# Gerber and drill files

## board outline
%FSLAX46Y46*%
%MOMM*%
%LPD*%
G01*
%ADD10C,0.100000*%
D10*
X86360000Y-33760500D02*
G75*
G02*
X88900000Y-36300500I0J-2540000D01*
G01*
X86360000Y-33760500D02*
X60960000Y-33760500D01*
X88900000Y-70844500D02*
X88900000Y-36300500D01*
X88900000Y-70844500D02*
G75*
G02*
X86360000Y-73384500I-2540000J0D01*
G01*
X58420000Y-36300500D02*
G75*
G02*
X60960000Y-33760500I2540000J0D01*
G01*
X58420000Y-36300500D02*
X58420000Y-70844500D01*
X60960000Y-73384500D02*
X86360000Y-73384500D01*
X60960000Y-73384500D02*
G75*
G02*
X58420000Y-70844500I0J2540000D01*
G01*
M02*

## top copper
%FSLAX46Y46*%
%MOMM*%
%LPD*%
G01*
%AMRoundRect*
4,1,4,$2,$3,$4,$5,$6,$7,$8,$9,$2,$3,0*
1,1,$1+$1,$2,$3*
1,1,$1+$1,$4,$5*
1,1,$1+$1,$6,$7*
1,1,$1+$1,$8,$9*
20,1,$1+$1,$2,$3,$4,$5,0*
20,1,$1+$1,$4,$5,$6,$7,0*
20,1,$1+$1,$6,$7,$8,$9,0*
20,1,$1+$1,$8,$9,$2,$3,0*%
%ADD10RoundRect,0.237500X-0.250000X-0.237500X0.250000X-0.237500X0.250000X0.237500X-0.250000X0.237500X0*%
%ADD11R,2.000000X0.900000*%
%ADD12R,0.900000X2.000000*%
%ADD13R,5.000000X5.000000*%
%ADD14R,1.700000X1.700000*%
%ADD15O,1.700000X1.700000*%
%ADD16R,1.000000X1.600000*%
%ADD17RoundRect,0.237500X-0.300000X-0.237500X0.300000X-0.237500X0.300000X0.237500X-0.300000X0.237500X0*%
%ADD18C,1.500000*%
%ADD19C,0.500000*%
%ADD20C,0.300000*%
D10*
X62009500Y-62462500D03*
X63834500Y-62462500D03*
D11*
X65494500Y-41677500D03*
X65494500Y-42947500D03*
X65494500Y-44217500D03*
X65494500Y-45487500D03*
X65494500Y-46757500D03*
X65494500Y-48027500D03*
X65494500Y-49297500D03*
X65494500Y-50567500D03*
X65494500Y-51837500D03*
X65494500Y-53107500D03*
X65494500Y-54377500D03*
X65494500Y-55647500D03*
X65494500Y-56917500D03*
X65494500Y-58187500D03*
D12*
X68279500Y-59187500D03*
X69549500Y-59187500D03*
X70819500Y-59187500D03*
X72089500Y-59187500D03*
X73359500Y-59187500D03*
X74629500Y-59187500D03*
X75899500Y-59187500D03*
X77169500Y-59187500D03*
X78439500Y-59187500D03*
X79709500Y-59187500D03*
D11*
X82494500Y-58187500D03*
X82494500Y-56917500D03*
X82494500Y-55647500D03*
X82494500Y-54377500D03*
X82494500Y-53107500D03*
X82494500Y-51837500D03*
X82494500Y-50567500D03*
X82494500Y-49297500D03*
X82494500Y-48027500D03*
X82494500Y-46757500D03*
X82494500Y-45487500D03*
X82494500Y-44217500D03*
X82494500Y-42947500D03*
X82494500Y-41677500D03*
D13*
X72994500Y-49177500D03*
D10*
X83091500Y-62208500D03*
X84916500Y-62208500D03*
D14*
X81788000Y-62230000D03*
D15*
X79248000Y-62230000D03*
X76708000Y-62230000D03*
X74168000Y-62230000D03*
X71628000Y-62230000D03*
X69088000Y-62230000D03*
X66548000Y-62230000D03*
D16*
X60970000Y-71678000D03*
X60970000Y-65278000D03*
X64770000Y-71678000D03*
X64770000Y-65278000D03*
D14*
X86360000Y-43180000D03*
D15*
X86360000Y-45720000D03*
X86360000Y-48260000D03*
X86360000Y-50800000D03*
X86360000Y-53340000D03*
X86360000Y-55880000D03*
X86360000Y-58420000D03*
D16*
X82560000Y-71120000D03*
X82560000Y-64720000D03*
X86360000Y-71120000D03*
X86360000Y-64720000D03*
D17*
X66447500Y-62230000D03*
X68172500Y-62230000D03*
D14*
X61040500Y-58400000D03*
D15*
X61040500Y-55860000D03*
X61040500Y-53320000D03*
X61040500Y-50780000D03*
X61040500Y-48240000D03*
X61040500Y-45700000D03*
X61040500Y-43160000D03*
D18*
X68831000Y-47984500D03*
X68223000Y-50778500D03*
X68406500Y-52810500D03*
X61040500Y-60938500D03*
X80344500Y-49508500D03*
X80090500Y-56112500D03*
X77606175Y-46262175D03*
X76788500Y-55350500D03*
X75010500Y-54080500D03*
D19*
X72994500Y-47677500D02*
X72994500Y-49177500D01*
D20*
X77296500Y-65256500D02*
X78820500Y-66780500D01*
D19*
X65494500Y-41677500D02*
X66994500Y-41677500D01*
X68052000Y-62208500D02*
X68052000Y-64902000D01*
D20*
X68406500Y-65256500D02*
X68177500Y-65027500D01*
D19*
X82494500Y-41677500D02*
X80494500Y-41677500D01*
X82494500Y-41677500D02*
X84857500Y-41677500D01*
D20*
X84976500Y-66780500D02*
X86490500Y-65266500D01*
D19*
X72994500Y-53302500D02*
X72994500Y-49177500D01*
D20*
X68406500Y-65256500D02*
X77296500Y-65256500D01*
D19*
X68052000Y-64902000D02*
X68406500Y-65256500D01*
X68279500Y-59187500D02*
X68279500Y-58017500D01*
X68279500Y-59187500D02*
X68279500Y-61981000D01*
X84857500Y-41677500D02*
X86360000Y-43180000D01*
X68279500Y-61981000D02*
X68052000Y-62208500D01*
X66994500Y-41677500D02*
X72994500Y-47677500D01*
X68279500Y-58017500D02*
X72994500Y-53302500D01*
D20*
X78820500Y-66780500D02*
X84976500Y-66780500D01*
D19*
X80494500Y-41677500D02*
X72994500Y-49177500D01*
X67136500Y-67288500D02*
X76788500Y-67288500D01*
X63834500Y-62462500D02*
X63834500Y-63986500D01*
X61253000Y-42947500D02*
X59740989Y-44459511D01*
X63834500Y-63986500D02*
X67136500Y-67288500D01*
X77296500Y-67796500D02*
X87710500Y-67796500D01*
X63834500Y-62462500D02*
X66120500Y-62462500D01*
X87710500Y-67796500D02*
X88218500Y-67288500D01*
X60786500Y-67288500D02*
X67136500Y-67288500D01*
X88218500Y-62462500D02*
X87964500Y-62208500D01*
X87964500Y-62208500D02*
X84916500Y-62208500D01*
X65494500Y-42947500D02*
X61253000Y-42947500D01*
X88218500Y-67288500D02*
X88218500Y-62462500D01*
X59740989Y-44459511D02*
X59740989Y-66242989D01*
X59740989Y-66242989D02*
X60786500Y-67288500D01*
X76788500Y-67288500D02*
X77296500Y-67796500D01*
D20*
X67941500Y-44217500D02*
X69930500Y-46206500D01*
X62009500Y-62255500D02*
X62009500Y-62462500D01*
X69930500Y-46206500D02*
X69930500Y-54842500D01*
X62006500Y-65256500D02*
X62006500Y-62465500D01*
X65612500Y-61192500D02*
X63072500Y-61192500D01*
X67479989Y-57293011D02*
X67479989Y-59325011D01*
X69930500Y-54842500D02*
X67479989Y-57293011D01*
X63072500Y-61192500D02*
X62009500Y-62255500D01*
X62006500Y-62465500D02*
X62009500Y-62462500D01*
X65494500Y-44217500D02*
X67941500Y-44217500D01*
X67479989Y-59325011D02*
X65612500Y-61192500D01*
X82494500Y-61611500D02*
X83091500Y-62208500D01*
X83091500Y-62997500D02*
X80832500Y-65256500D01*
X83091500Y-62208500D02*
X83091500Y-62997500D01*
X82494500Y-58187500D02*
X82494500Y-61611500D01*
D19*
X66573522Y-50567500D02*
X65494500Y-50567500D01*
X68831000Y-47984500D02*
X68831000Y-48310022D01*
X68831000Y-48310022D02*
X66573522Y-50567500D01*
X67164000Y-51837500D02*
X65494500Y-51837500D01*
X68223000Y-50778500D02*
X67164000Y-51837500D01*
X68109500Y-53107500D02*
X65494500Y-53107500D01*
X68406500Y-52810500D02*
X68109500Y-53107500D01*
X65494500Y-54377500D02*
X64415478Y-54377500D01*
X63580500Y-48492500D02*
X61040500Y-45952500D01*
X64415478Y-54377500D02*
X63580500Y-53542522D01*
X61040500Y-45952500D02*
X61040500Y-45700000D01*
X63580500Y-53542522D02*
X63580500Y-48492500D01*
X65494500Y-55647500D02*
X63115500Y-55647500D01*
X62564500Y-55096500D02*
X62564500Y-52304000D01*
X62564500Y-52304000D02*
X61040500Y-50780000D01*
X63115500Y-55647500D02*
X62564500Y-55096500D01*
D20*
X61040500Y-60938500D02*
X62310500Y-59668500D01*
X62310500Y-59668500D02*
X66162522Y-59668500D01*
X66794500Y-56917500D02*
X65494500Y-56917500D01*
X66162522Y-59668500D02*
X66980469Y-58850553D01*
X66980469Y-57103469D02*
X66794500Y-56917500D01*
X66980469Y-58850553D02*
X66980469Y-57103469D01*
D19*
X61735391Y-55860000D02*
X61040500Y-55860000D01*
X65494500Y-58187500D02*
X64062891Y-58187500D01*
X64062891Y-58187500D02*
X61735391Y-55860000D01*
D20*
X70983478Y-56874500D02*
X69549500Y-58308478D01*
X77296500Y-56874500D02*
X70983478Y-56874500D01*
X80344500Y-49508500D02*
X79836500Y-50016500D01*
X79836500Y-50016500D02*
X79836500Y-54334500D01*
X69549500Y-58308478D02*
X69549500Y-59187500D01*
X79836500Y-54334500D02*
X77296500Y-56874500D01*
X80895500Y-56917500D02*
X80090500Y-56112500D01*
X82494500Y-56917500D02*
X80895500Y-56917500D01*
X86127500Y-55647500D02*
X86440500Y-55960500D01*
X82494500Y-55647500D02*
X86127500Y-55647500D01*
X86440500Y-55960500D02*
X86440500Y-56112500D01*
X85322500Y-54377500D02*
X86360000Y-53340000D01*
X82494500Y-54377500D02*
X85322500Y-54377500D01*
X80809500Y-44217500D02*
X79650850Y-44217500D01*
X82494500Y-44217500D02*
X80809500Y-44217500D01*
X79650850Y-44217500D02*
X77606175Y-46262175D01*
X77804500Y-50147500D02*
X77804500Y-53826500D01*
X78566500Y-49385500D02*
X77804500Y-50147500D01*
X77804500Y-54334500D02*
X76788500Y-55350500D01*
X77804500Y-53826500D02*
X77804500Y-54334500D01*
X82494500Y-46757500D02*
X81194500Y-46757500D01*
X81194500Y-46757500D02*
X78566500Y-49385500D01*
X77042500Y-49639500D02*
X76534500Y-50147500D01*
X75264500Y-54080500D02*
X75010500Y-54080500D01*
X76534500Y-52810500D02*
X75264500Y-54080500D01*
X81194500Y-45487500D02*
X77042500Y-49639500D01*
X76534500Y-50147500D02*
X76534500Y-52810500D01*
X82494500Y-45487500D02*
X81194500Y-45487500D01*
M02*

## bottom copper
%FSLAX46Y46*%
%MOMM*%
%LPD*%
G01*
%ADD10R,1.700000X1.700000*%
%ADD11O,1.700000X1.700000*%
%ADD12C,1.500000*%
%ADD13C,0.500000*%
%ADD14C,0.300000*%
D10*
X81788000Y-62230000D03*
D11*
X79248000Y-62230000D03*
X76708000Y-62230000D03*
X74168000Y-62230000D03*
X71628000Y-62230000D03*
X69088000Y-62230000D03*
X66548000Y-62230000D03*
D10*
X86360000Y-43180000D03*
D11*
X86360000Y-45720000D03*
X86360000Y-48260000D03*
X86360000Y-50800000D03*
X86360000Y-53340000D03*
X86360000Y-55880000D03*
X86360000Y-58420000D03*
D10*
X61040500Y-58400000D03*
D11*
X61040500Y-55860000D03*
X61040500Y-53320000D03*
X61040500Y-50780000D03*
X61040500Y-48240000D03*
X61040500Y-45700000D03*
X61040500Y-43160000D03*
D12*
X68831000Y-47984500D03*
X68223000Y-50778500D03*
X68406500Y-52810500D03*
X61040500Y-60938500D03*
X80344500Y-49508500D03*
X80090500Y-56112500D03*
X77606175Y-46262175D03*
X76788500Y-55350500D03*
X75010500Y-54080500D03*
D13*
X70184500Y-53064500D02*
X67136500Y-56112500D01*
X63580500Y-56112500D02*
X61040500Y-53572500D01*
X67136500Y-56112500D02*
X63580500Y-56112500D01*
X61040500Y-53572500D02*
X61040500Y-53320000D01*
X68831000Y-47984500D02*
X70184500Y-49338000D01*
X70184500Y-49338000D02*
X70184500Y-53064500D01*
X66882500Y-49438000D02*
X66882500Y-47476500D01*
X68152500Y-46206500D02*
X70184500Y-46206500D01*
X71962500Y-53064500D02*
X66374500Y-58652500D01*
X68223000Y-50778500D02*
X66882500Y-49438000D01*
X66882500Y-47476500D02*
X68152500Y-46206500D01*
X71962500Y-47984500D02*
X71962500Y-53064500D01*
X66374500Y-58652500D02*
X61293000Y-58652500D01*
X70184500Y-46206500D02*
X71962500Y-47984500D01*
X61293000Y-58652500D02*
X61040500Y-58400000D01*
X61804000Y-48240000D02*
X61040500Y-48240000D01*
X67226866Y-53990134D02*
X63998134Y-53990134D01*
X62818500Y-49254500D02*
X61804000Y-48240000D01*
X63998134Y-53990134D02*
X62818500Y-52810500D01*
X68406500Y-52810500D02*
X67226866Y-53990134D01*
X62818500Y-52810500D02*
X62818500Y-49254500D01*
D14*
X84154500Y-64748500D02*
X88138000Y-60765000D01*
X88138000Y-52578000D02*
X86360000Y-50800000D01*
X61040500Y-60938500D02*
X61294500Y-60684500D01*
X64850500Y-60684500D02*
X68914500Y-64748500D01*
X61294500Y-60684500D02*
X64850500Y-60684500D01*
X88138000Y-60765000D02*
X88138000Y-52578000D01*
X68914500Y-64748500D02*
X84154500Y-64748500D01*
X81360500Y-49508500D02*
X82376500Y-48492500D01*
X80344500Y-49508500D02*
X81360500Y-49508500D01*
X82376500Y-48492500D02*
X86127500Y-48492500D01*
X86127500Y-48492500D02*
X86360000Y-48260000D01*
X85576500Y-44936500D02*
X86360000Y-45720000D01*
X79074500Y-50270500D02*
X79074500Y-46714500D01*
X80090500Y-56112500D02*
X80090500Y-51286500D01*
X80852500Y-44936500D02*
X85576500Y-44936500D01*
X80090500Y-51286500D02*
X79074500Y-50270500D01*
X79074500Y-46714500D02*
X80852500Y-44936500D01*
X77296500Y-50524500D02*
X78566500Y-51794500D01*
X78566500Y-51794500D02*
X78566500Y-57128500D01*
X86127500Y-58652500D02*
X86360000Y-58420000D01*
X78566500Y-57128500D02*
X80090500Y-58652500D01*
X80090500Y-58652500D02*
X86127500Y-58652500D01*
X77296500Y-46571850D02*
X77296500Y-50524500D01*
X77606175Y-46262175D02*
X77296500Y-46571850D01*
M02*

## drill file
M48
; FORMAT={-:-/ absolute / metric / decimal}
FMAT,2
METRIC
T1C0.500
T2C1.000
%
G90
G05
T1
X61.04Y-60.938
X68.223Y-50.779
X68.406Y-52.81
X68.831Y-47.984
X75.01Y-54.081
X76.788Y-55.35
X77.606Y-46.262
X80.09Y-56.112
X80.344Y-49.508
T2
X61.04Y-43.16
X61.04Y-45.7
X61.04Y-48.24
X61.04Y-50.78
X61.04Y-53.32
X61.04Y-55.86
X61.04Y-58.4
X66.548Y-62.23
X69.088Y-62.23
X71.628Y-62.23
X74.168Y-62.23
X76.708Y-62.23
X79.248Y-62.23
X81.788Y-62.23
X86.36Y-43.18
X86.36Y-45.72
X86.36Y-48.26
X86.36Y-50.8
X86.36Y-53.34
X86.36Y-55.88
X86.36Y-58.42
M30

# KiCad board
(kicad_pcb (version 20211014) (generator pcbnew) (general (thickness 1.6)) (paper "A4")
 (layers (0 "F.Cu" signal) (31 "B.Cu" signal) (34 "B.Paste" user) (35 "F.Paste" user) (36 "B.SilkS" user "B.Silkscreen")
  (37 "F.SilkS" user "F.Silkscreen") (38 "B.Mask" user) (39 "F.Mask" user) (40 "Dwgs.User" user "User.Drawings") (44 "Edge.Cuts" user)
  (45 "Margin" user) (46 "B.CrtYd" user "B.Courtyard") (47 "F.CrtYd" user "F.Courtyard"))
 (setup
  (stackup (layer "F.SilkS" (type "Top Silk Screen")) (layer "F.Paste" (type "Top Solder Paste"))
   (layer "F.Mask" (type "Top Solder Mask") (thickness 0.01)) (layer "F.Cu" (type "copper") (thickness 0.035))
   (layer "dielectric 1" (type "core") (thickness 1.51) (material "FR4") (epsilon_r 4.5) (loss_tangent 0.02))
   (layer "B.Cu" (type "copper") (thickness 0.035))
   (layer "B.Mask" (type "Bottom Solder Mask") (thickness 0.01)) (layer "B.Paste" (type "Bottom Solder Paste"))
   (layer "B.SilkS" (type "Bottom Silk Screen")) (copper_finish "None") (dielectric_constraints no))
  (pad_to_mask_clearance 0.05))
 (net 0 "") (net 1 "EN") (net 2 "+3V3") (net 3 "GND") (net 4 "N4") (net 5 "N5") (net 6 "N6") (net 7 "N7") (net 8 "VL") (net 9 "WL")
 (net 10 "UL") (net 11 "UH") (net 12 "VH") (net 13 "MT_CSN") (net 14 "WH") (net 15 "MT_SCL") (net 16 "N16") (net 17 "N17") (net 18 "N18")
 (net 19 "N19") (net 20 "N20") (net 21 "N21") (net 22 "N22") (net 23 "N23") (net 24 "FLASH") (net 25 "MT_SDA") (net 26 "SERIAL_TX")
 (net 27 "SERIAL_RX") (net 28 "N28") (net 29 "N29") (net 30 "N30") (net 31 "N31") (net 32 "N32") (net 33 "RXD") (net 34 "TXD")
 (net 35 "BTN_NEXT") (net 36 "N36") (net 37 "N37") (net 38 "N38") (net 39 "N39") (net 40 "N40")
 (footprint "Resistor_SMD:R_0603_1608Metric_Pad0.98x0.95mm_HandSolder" (layer "F.Cu") (at 62.922 62.4625)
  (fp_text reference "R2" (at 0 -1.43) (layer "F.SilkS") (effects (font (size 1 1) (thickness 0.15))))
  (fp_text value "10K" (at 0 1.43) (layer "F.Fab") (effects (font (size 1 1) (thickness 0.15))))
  (pad "1" smd roundrect (at -0.9125 0) (size 0.975 0.95) (layers "F.Cu" "F.Paste" "F.Mask") (roundrect_rratio 0.25) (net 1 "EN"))
  (pad "2" smd roundrect (at 0.9125 0) (size 0.975 0.95) (layers "F.Cu" "F.Paste" "F.Mask") (roundrect_rratio 0.25) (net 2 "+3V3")))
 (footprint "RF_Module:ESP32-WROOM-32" (layer "F.Cu") (at 73.9945 49.9325)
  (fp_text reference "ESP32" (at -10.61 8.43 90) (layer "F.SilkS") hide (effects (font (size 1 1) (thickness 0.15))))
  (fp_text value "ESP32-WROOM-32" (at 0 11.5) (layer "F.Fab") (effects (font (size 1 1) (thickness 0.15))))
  (pad "1" smd rect (at -8.5 -8.255) (size 2 0.9) (layers "F.Cu" "F.Paste" "F.Mask") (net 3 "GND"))
  (pad "2" smd rect (at -8.5 -6.985) (size 2 0.9) (layers "F.Cu" "F.Paste" "F.Mask") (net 2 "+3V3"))
  (pad "3" smd rect (at -8.5 -5.715) (size 2 0.9) (layers "F.Cu" "F.Paste" "F.Mask") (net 1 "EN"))
  (pad "4" smd rect (at -8.5 -4.445) (size 2 0.9) (layers "F.Cu" "F.Paste" "F.Mask") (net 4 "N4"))
  (pad "5" smd rect (at -8.5 -3.175) (size 2 0.9) (layers "F.Cu" "F.Paste" "F.Mask") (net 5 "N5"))
  (pad "6" smd rect (at -8.5 -1.905) (size 2 0.9) (layers "F.Cu" "F.Paste" "F.Mask") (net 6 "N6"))
  (pad "7" smd rect (at -8.5 -0.635) (size 2 0.9) (layers "F.Cu" "F.Paste" "F.Mask") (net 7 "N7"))
  (pad "8" smd rect (at -8.5 0.635) (size 2 0.9) (layers "F.Cu" "F.Paste" "F.Mask") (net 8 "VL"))
  (pad "9" smd rect (at -8.5 1.905) (size 2 0.9) (layers "F.Cu" "F.Paste" "F.Mask") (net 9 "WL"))
  (pad "10" smd rect (at -8.5 3.175) (size 2 0.9) (layers "F.Cu" "F.Paste" "F.Mask") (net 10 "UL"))
  (pad "11" smd rect (at -8.5 4.445) (size 2 0.9) (layers "F.Cu" "F.Paste" "F.Mask") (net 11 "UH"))
  (pad "12" smd rect (at -8.5 5.715) (size 2 0.9) (layers "F.Cu" "F.Paste" "F.Mask") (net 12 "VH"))
  (pad "13" smd rect (at -8.5 6.985) (size 2 0.9) (layers "F.Cu" "F.Paste" "F.Mask") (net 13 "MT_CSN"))
  (pad "14" smd rect (at -8.5 8.255) (size 2 0.9) (layers "F.Cu" "F.Paste" "F.Mask") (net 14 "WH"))
  (pad "15" smd rect (at -5.715 9.255 90) (size 2 0.9) (layers "F.Cu" "F.Paste" "F.Mask") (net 3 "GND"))
  (pad "16" smd rect (at -4.445 9.255 90) (size 2 0.9) (layers "F.Cu" "F.Paste" "F.Mask") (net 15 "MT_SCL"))
  (pad "17" smd rect (at -3.175 9.255 90) (size 2 0.9) (layers "F.Cu" "F.Paste" "F.Mask") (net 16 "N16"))
  (pad "18" smd rect (at -1.905 9.255 90) (size 2 0.9) (layers "F.Cu" "F.Paste" "F.Mask") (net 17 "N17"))
  (pad "19" smd rect (at -0.635 9.255 90) (size 2 0.9) (layers "F.Cu" "F.Paste" "F.Mask") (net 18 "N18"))
  (pad "20" smd rect (at 0.635 9.255 90) (size 2 0.9) (layers "F.Cu" "F.Paste" "F.Mask") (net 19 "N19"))
  (pad "21" smd rect (at 1.905 9.255 90) (size 2 0.9) (layers "F.Cu" "F.Paste" "F.Mask") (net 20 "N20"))
  (pad "22" smd rect (at 3.175 9.255 90) (size 2 0.9) (layers "F.Cu" "F.Paste" "F.Mask") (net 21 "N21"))
  (pad "23" smd rect (at 4.445 9.255 90) (size 2 0.9) (layers "F.Cu" "F.Paste" "F.Mask") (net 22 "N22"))
  (pad "24" smd rect (at 5.715 9.255 90) (size 2 0.9) (layers "F.Cu" "F.Paste" "F.Mask") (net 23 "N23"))
  (pad "25" smd rect (at 8.5 8.255) (size 2 0.9) (layers "F.Cu" "F.Paste" "F.Mask") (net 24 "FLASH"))
  (pad "26" smd rect (at 8.5 6.985) (size 2 0.9) (layers "F.Cu" "F.Paste" "F.Mask") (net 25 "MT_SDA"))
  (pad "27" smd rect (at 8.5 5.715) (size 2 0.9) (layers "F.Cu" "F.Paste" "F.Mask") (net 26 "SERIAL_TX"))
  (pad "28" smd rect (at 8.5 4.445) (size 2 0.9) (layers "F.Cu" "F.Paste" "F.Mask") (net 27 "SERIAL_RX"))
  (pad "29" smd rect (at 8.5 3.175) (size 2 0.9) (layers "F.Cu" "F.Paste" "F.Mask") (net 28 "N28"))
  (pad "30" smd rect (at 8.5 1.905) (size 2 0.9) (layers "F.Cu" "F.Paste" "F.Mask") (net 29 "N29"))
  (pad "31" smd rect (at 8.5 0.635) (size 2 0.9) (layers "F.Cu" "F.Paste" "F.Mask") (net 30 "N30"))
  (pad "32" smd rect (at 8.5 -0.635) (size 2 0.9) (layers "F.Cu" "F.Paste" "F.Mask") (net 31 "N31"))
  (pad "33" smd rect (at 8.5 -1.905) (size 2 0.9) (layers "F.Cu" "F.Paste" "F.Mask") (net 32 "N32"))
  (pad "34" smd rect (at 8.5 -3.175) (size 2 0.9) (layers "F.Cu" "F.Paste" "F.Mask") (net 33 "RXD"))
  (pad "35" smd rect (at 8.5 -4.445) (size 2 0.9) (layers "F.Cu" "F.Paste" "F.Mask") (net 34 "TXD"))
  (pad "36" smd rect (at 8.5 -5.715) (size 2 0.9) (layers "F.Cu" "F.Paste" "F.Mask") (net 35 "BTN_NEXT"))
  (pad "37" smd rect (at 8.5 -6.985) (size 2 0.9) (layers "F.Cu" "F.Paste" "F.Mask") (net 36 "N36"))
  (pad "38" smd rect (at 8.5 -8.255) (size 2 0.9) (layers "F.Cu" "F.Paste" "F.Mask") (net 3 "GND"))
  (pad "39" smd rect (at -1 -0.755) (size 5 5) (layers "F.Cu" "F.Paste" "F.Mask") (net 3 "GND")))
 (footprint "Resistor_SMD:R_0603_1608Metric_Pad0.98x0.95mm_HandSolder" (layer "F.Cu") (at 84.004 62.2085)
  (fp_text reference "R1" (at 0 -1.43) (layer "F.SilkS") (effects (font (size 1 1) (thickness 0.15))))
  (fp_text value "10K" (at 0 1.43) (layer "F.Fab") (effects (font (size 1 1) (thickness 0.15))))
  (pad "1" smd roundrect (at -0.9125 0) (size 0.975 0.95) (layers "F.Cu" "F.Paste" "F.Mask") (roundrect_rratio 0.25) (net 24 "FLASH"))
  (pad "2" smd roundrect (at 0.9125 0) (size 0.975 0.95) (layers "F.Cu" "F.Paste" "F.Mask") (roundrect_rratio 0.25) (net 2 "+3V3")))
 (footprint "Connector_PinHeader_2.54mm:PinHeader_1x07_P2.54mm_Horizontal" (layer "F.Cu") (at 81.788 62.23 -90)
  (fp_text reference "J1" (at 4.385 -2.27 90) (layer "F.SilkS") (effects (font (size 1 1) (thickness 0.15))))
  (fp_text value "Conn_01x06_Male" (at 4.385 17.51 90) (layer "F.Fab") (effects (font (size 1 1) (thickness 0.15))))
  (pad "1" thru_hole rect (at 0 0 270) (size 1.7 1.7) (drill 1) (layers *.Cu *.Mask) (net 2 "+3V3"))
  (pad "2" thru_hole oval (at 0 2.54 270) (size 1.7 1.7) (drill 1) (layers *.Cu *.Mask) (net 34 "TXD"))
  (pad "3" thru_hole oval (at 0 5.08 270) (size 1.7 1.7) (drill 1) (layers *.Cu *.Mask) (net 33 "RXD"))
  (pad "4" thru_hole oval (at 0 7.62 270) (size 1.7 1.7) (drill 1) (layers *.Cu *.Mask) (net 1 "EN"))
  (pad "5" thru_hole oval (at 0 10.16 270) (size 1.7 1.7) (drill 1) (layers *.Cu *.Mask) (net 24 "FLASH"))
  (pad "6" thru_hole oval (at 0 12.7 270) (size 1.7 1.7) (drill 1) (layers *.Cu *.Mask) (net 3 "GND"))
  (pad "7" thru_hole oval (at 0 15.24 270) (size 1.7 1.7) (drill 1) (layers *.Cu *.Mask)))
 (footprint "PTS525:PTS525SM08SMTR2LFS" (layer "F.Cu") (at 62.87 69.128 90)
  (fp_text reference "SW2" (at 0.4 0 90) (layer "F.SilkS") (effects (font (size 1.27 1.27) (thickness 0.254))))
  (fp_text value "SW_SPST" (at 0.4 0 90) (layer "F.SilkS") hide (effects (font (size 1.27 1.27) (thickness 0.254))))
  (pad "1" smd rect locked (at -2.55 -1.9 180) (size 1 1.6) (layers "F.Cu" "F.Paste" "F.Mask") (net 1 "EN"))
  (pad "2" smd rect locked (at 3.85 -1.9 180) (size 1 1.6) (layers "F.Cu" "F.Paste" "F.Mask") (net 3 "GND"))
  (pad "3" smd rect locked (at -2.55 1.9 180) (size 1 1.6) (layers "F.Cu" "F.Paste" "F.Mask") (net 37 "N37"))
  (pad "4" smd rect locked (at 3.85 1.9 180) (size 1 1.6) (layers "F.Cu" "F.Paste" "F.Mask") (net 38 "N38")))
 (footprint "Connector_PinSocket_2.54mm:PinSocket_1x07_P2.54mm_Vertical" (layer "F.Cu") (at 86.36 43.18)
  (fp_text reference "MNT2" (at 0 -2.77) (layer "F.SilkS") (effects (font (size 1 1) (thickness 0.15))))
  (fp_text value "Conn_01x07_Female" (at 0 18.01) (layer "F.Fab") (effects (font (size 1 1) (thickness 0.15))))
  (pad "1" thru_hole rect (at 0 0) (size 1.7 1.7) (drill 1) (layers *.Cu *.Mask) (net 3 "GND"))
  (pad "2" thru_hole oval (at 0 2.54) (size 1.7 1.7) (drill 1) (layers *.Cu *.Mask) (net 25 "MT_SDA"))
  (pad "3" thru_hole oval (at 0 5.08) (size 1.7 1.7) (drill 1) (layers *.Cu *.Mask) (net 15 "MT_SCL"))
  (pad "4" thru_hole oval (at 0 7.62) (size 1.7 1.7) (drill 1) (layers *.Cu *.Mask) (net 13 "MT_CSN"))
  (pad "5" thru_hole oval (at 0 10.16) (size 1.7 1.7) (drill 1) (layers *.Cu *.Mask) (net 27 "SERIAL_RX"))
  (pad "6" thru_hole oval (at 0 12.7) (size 1.7 1.7) (drill 1) (layers *.Cu *.Mask) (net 26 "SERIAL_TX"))
  (pad "7" thru_hole oval (at 0 15.24) (size 1.7 1.7) (drill 1) (layers *.Cu *.Mask) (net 35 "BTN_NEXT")))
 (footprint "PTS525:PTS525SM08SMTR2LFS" (layer "F.Cu") (at 84.46 68.57 90)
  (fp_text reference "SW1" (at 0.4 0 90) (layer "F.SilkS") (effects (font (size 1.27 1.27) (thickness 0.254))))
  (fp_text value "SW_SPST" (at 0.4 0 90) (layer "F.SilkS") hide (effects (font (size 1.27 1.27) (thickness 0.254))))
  (pad "1" smd rect locked (at -2.55 -1.9 180) (size 1 1.6) (layers "F.Cu" "F.Paste" "F.Mask") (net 24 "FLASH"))
  (pad "2" smd rect locked (at 3.85 -1.9 180) (size 1 1.6) (layers "F.Cu" "F.Paste" "F.Mask") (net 3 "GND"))
  (pad "3" smd rect locked (at -2.55 1.9 180) (size 1 1.6) (layers "F.Cu" "F.Paste" "F.Mask") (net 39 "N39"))
  (pad "4" smd rect locked (at 3.85 1.9 180) (size 1 1.6) (layers "F.Cu" "F.Paste" "F.Mask") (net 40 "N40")))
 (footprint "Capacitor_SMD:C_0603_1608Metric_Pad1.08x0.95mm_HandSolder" (layer "F.Cu") (at 67.31 62.23)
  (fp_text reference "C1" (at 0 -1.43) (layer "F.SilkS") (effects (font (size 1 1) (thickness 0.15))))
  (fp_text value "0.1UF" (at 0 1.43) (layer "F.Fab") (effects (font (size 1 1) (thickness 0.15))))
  (pad "1" smd roundrect (at -0.8625 0) (size 1.075 0.95) (layers "F.Cu" "F.Paste" "F.Mask") (roundrect_rratio 0.25) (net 2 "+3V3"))
  (pad "2" smd roundrect (at 0.8625 0) (size 1.075 0.95) (layers "F.Cu" "F.Paste" "F.Mask") (roundrect_rratio 0.25) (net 3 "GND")))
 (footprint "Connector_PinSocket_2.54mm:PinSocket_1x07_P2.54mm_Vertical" (layer "F.Cu") (at 61.0405 58.4 180)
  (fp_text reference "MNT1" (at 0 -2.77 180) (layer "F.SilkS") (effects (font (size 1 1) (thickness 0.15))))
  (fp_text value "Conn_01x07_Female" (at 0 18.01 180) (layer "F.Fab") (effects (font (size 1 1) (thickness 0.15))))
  (pad "1" thru_hole rect (at 0 0 180) (size 1.7 1.7) (drill 1) (layers *.Cu *.Mask) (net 9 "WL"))
  (pad "2" thru_hole oval (at 0 2.54 180) (size 1.7 1.7) (drill 1) (layers *.Cu *.Mask) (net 14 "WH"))
  (pad "3" thru_hole oval (at 0 5.08 180) (size 1.7 1.7) (drill 1) (layers *.Cu *.Mask) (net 8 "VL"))
  (pad "4" thru_hole oval (at 0 7.62 180) (size 1.7 1.7) (drill 1) (layers *.Cu *.Mask) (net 12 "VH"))
  (pad "5" thru_hole oval (at 0 10.16 180) (size 1.7 1.7) (drill 1) (layers *.Cu *.Mask) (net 10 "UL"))
  (pad "6" thru_hole oval (at 0 12.7 180) (size 1.7 1.7) (drill 1) (layers *.Cu *.Mask) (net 11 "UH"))
  (pad "7" thru_hole oval (at 0 15.24 180) (size 1.7 1.7) (drill 1) (layers *.Cu *.Mask) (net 2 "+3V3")))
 (gr_arc (start 86.36 33.7605) (mid 88.156051 34.504449) (end 88.9 36.3005) (layer "Edge.Cuts") (width 0.1))
 (gr_line (start 86.36 33.7605) (end 60.96 33.7605) (layer "Edge.Cuts") (width 0.1))
 (gr_line (start 88.9 70.8445) (end 88.9 36.3005) (layer "Edge.Cuts") (width 0.1))
 (gr_arc (start 88.9 70.8445) (mid 88.156051 72.640551) (end 86.36 73.3845) (layer "Edge.Cuts") (width 0.1))
 (gr_arc (start 58.42 36.3005) (mid 59.163949 34.504449) (end 60.96 33.7605) (layer "Edge.Cuts") (width 0.1))
 (gr_line (start 58.42 36.3005) (end 58.42 70.8445) (layer "Edge.Cuts") (width 0.1))
 (gr_line (start 60.96 73.3845) (end 86.36 73.3845) (layer "Edge.Cuts") (width 0.1))
 (gr_arc (start 60.96 73.3845) (mid 59.163949 72.640551) (end 58.42 70.8445) (layer "Edge.Cuts") (width 0.1))
 (segment (start 72.9945 47.6775) (end 72.9945 49.1775) (width 0.5) (layer "F.Cu") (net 3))
 (segment (start 77.2965 65.2565) (end 78.8205 66.7805) (width 0.3) (layer "F.Cu") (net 3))
 (segment (start 65.4945 41.6775) (end 66.9945 41.6775) (width 0.5) (layer "F.Cu") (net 3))
 (segment (start 68.052 62.2085) (end 68.052 64.902) (width 0.5) (layer "F.Cu") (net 3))
 (segment (start 68.4065 65.2565) (end 68.1775 65.0275) (width 0.3) (layer "F.Cu") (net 3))
 (segment (start 82.4945 41.6775) (end 80.4945 41.6775) (width 0.5) (layer "F.Cu") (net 3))
 (segment (start 82.4945 41.6775) (end 84.8575 41.6775) (width 0.5) (layer "F.Cu") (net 3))
 (segment (start 84.9765 66.7805) (end 86.4905 65.2665) (width 0.3) (layer "F.Cu") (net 3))
 (segment (start 72.9945 53.3025) (end 72.9945 49.1775) (width 0.5) (layer "F.Cu") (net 3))
 (segment (start 68.4065 65.2565) (end 77.2965 65.2565) (width 0.3) (layer "F.Cu") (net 3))
 (segment (start 68.052 64.902) (end 68.4065 65.2565) (width 0.5) (layer "F.Cu") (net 3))
 (segment (start 68.2795 59.1875) (end 68.2795 58.0175) (width 0.5) (layer "F.Cu") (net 3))
 (segment (start 68.2795 59.1875) (end 68.2795 61.981) (width 0.5) (layer "F.Cu") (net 3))
 (segment (start 84.8575 41.6775) (end 86.36 43.18) (width 0.5) (layer "F.Cu") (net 3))
 (segment (start 68.2795 61.981) (end 68.052 62.2085) (width 0.5) (layer "F.Cu") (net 3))
 (segment (start 66.9945 41.6775) (end 72.9945 47.6775) (width 0.5) (layer "F.Cu") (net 3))
 (segment (start 68.2795 58.0175) (end 72.9945 53.3025) (width 0.5) (layer "F.Cu") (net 3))
 (segment (start 78.8205 66.7805) (end 84.9765 66.7805) (width 0.3) (layer "F.Cu") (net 3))
 (segment (start 80.4945 41.6775) (end 72.9945 49.1775) (width 0.5) (layer "F.Cu") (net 3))
 (segment (start 67.1365 67.2885) (end 76.7885 67.2885) (width 0.5) (layer "F.Cu") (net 2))
 (segment (start 63.8345 62.4625) (end 63.8345 63.9865) (width 0.5) (layer "F.Cu") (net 2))
 (segment (start 61.253 42.9475) (end 59.740989 44.459511) (width 0.5) (layer "F.Cu") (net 2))
 (segment (start 63.8345 63.9865) (end 67.1365 67.2885) (width 0.5) (layer "F.Cu") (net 2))
 (segment (start 77.2965 67.7965) (end 87.7105 67.7965) (width 0.5) (layer "F.Cu") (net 2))
 (segment (start 63.8345 62.4625) (end 66.1205 62.4625) (width 0.5) (layer "F.Cu") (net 2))
 (segment (start 87.7105 67.7965) (end 88.2185 67.2885) (width 0.5) (layer "F.Cu") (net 2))
 (segment (start 60.7865 67.2885) (end 67.1365 67.2885) (width 0.5) (layer "F.Cu") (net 2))
 (segment (start 88.2185 62.4625) (end 87.9645 62.2085) (width 0.5) (layer "F.Cu") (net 2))
 (segment (start 87.9645 62.2085) (end 84.9165 62.2085) (width 0.5) (layer "F.Cu") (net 2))
 (segment (start 65.4945 42.9475) (end 61.253 42.9475) (width 0.5) (layer "F.Cu") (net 2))
 (segment (start 88.2185 67.2885) (end 88.2185 62.4625) (width 0.5) (layer "F.Cu") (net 2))
 (segment (start 59.740989 44.459511) (end 59.740989 66.242989) (width 0.5) (layer "F.Cu") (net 2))
 (segment (start 59.740989 66.242989) (end 60.7865 67.2885) (width 0.5) (layer "F.Cu") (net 2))
 (segment (start 76.7885 67.2885) (end 77.2965 67.7965) (width 0.5) (layer "F.Cu") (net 2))
 (segment (start 67.9415 44.2175) (end 69.9305 46.2065) (width 0.3) (layer "F.Cu") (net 1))
 (segment (start 62.0095 62.2555) (end 62.0095 62.4625) (width 0.3) (layer "F.Cu") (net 1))
 (segment (start 69.9305 46.2065) (end 69.9305 54.8425) (width 0.3) (layer "F.Cu") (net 1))
 (segment (start 62.0065 65.2565) (end 62.0065 62.4655) (width 0.3) (layer "F.Cu") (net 1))
 (segment (start 65.6125 61.1925) (end 63.0725 61.1925) (width 0.3) (layer "F.Cu") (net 1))
 (segment (start 67.479989 57.293011) (end 67.479989 59.325011) (width 0.3) (layer "F.Cu") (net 1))
 (segment (start 69.9305 54.8425) (end 67.479989 57.293011) (width 0.3) (layer "F.Cu") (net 1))
 (segment (start 63.0725 61.1925) (end 62.0095 62.2555) (width 0.3) (layer "F.Cu") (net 1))
 (segment (start 62.0065 62.4655) (end 62.0095 62.4625) (width 0.3) (layer "F.Cu") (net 1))
 (segment (start 65.4945 44.2175) (end 67.9415 44.2175) (width 0.3) (layer "F.Cu") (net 1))
 (segment (start 67.479989 59.325011) (end 65.6125 61.1925) (width 0.3) (layer "F.Cu") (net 1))
 (segment (start 82.4945 61.6115) (end 83.0915 62.2085) (width 0.3) (layer "F.Cu") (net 24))
 (segment (start 83.0915 62.9975) (end 80.8325 65.2565) (width 0.3) (layer "F.Cu") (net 24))
 (segment (start 83.0915 62.2085) (end 83.0915 62.9975) (width 0.3) (layer "F.Cu") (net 24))
 (segment (start 82.4945 58.1875) (end 82.4945 61.6115) (width 0.3) (layer "F.Cu") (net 24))
 (segment (start 66.573522 50.5675) (end 65.4945 50.5675) (width 0.5) (layer "F.Cu") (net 8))
 (segment (start 68.831 47.9845) (end 68.831 48.310022) (width 0.5) (layer "F.Cu") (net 8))
 (segment (start 68.831 48.310022) (end 66.573522 50.5675) (width 0.5) (layer "F.Cu") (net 8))
 (via (at 68.831 47.9845) (size 1.5) (drill 0.5) (layers "F.Cu" "B.Cu") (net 8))
 (segment (start 70.1845 53.0645) (end 67.1365 56.1125) (width 0.5) (layer "B.Cu") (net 8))
 (segment (start 63.5805 56.1125) (end 61.0405 53.5725) (width 0.5) (layer "B.Cu") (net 8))
 (segment (start 67.1365 56.1125) (end 63.5805 56.1125) (width 0.5) (layer "B.Cu") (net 8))
 (segment (start 61.0405 53.5725) (end 61.0405 53.32) (width 0.5) (layer "B.Cu") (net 8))
 (segment (start 68.831 47.9845) (end 70.1845 49.338) (width 0.5) (layer "B.Cu") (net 8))
 (segment (start 70.1845 49.338) (end 70.1845 53.0645) (width 0.5) (layer "B.Cu") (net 8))
 (segment (start 67.164 51.8375) (end 65.4945 51.8375) (width 0.5) (layer "F.Cu") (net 9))
 (segment (start 68.223 50.7785) (end 67.164 51.8375) (width 0.5) (layer "F.Cu") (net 9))
 (via (at 68.223 50.7785) (size 1.5) (drill 0.5) (layers "F.Cu" "B.Cu") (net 9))
 (segment (start 66.8825 49.438) (end 66.8825 47.4765) (width 0.5) (layer "B.Cu") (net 9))
 (segment (start 68.1525 46.2065) (end 70.1845 46.2065) (width 0.5) (layer "B.Cu") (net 9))
 (segment (start 71.9625 53.0645) (end 66.3745 58.6525) (width 0.5) (layer "B.Cu") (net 9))
 (segment (start 68.223 50.7785) (end 66.8825 49.438) (width 0.5) (layer "B.Cu") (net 9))
 (segment (start 66.8825 47.4765) (end 68.1525 46.2065) (width 0.5) (layer "B.Cu") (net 9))
 (segment (start 71.9625 47.9845) (end 71.9625 53.0645) (width 0.5) (layer "B.Cu") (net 9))
 (segment (start 66.3745 58.6525) (end 61.293 58.6525) (width 0.5) (layer "B.Cu") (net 9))
 (segment (start 70.1845 46.2065) (end 71.9625 47.9845) (width 0.5) (layer "B.Cu") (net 9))
 (segment (start 61.293 58.6525) (end 61.0405 58.4) (width 0.5) (layer "B.Cu") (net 9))
 (segment (start 68.1095 53.1075) (end 65.4945 53.1075) (width 0.5) (layer "F.Cu") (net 10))
 (segment (start 68.4065 52.8105) (end 68.1095 53.1075) (width 0.5) (layer "F.Cu") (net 10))
 (via (at 68.4065 52.8105) (size 1.5) (drill 0.5) (layers "F.Cu" "B.Cu") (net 10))
 (segment (start 61.804 48.24) (end 61.0405 48.24) (width 0.5) (layer "B.Cu") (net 10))
 (segment (start 67.226866 53.990134) (end 63.998134 53.990134) (width 0.5) (layer "B.Cu") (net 10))
 (segment (start 62.8185 49.2545) (end 61.804 48.24) (width 0.5) (layer "B.Cu") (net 10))
 (segment (start 63.998134 53.990134) (end 62.8185 52.8105) (width 0.5) (layer "B.Cu") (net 10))
 (segment (start 68.4065 52.8105) (end 67.226866 53.990134) (width 0.5) (layer "B.Cu") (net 10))
 (segment (start 62.8185 52.8105) (end 62.8185 49.2545) (width 0.5) (layer "B.Cu") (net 10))
 (segment (start 65.4945 54.3775) (end 64.415478 54.3775) (width 0.5) (layer "F.Cu") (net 11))
 (segment (start 63.5805 48.4925) (end 61.0405 45.9525) (width 0.5) (layer "F.Cu") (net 11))
 (segment (start 64.415478 54.3775) (end 63.5805 53.542522) (width 0.5) (layer "F.Cu") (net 11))
 (segment (start 61.0405 45.9525) (end 61.0405 45.7) (width 0.5) (layer "F.Cu") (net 11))
 (segment (start 63.5805 53.542522) (end 63.5805 48.4925) (width 0.5) (layer "F.Cu") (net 11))
 (segment (start 65.4945 55.6475) (end 63.1155 55.6475) (width 0.5) (layer "F.Cu") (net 12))
 (segment (start 62.5645 55.0965) (end 62.5645 52.304) (width 0.5) (layer "F.Cu") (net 12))
 (segment (start 62.5645 52.304) (end 61.0405 50.78) (width 0.5) (layer "F.Cu") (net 12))
 (segment (start 63.1155 55.6475) (end 62.5645 55.0965) (width 0.5) (layer "F.Cu") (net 12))
 (segment (start 61.0405 60.9385) (end 62.3105 59.6685) (width 0.3) (layer "F.Cu") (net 13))
 (segment (start 62.3105 59.6685) (end 66.162522 59.6685) (width 0.3) (layer "F.Cu") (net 13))
 (segment (start 66.7945 56.9175) (end 65.4945 56.9175) (width 0.3) (layer "F.Cu") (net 13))
 (segment (start 66.162522 59.6685) (end 66.980469 58.850553) (width 0.3) (layer "F.Cu") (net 13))
 (segment (start 66.980469 57.103469) (end 66.7945 56.9175) (width 0.3) (layer "F.Cu") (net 13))
 (segment (start 66.980469 58.850553) (end 66.980469 57.103469) (width 0.3) (layer "F.Cu") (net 13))
 (via (at 61.0405 60.9385) (size 1.5) (drill 0.5) (layers "F.Cu" "B.Cu") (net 13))
 (segment (start 84.1545 64.7485) (end 88.138 60.765) (width 0.3) (layer "B.Cu") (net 13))
 (segment (start 88.138 52.578) (end 86.36 50.8) (width 0.3) (layer "B.Cu") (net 13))
 (segment (start 61.0405 60.9385) (end 61.2945 60.6845) (width 0.3) (layer "B.Cu") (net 13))
 (segment (start 64.8505 60.6845) (end 68.9145 64.7485) (width 0.3) (layer "B.Cu") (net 13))
 (segment (start 61.2945 60.6845) (end 64.8505 60.6845) (width 0.3) (layer "B.Cu") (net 13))
 (segment (start 88.138 60.765) (end 88.138 52.578) (width 0.3) (layer "B.Cu") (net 13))
 (segment (start 68.9145 64.7485) (end 84.1545 64.7485) (width 0.3) (layer "B.Cu") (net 13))
 (segment (start 61.735391 55.86) (end 61.0405 55.86) (width 0.5) (layer "F.Cu") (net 14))
 (segment (start 65.4945 58.1875) (end 64.062891 58.1875) (width 0.5) (layer "F.Cu") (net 14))
 (segment (start 64.062891 58.1875) (end 61.735391 55.86) (width 0.5) (layer "F.Cu") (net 14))
 (segment (start 70.983478 56.8745) (end 69.5495 58.308478) (width 0.3) (layer "F.Cu") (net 15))
 (segment (start 77.2965 56.8745) (end 70.983478 56.8745) (width 0.3) (layer "F.Cu") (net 15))
 (segment (start 80.3445 49.5085) (end 79.8365 50.0165) (width 0.3) (layer "F.Cu") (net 15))
 (segment (start 79.8365 50.0165) (end 79.8365 54.3345) (width 0.3) (layer "F.Cu") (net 15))
 (segment (start 69.5495 58.308478) (end 69.5495 59.1875) (width 0.3) (layer "F.Cu") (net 15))
 (segment (start 79.8365 54.3345) (end 77.2965 56.8745) (width 0.3) (layer "F.Cu") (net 15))
 (via (at 80.3445 49.5085) (size 1.5) (drill 0.5) (layers "F.Cu" "B.Cu") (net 15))
 (segment (start 81.3605 49.5085) (end 82.3765 48.4925) (width 0.3) (layer "B.Cu") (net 15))
 (segment (start 80.3445 49.5085) (end 81.3605 49.5085) (width 0.3) (layer "B.Cu") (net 15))
 (segment (start 82.3765 48.4925) (end 86.1275 48.4925) (width 0.3) (layer "B.Cu") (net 15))
 (segment (start 86.1275 48.4925) (end 86.36 48.26) (width 0.3) (layer "B.Cu") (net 15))
 (segment (start 80.8955 56.9175) (end 80.0905 56.1125) (width 0.3) (layer "F.Cu") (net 25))
 (segment (start 82.4945 56.9175) (end 80.8955 56.9175) (width 0.3) (layer "F.Cu") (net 25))
 (via (at 80.0905 56.1125) (size 1.5) (drill 0.5) (layers "F.Cu" "B.Cu") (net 25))
 (segment (start 85.5765 44.9365) (end 86.36 45.72) (width 0.3) (layer "B.Cu") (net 25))
 (segment (start 79.0745 50.2705) (end 79.0745 46.7145) (width 0.3) (layer "B.Cu") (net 25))
 (segment (start 80.0905 56.1125) (end 80.0905 51.2865) (width 0.3) (layer "B.Cu") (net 25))
 (segment (start 80.8525 44.9365) (end 85.5765 44.9365) (width 0.3) (layer "B.Cu") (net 25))
 (segment (start 80.0905 51.2865) (end 79.0745 50.2705) (width 0.3) (layer "B.Cu") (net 25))
 (segment (start 79.0745 46.7145) (end 80.8525 44.9365) (width 0.3) (layer "B.Cu") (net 25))
 (segment (start 86.1275 55.6475) (end 86.4405 55.9605) (width 0.3) (layer "F.Cu") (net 26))
 (segment (start 82.4945 55.6475) (end 86.1275 55.6475) (width 0.3) (layer "F.Cu") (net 26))
 (segment (start 86.4405 55.9605) (end 86.4405 56.1125) (width 0.3) (layer "F.Cu") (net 26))
 (segment (start 85.3225 54.3775) (end 86.36 53.34) (width 0.3) (layer "F.Cu") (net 27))
 (segment (start 82.4945 54.3775) (end 85.3225 54.3775) (width 0.3) (layer "F.Cu") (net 27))
 (segment (start 80.8095 44.2175) (end 79.65085 44.2175) (width 0.3) (layer "F.Cu") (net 35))
 (segment (start 82.4945 44.2175) (end 80.8095 44.2175) (width 0.3) (layer "F.Cu") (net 35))
 (segment (start 79.65085 44.2175) (end 77.606175 46.262175) (width 0.3) (layer "F.Cu") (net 35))
 (via (at 77.606175 46.262175) (size 1.5) (drill 0.5) (layers "F.Cu" "B.Cu") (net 35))
 (segment (start 77.2965 50.5245) (end 78.5665 51.7945) (width 0.3) (layer "B.Cu") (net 35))
 (segment (start 78.5665 51.7945) (end 78.5665 57.1285) (width 0.3) (layer "B.Cu") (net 35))
 (segment (start 86.1275 58.6525) (end 86.36 58.42) (width 0.3) (layer "B.Cu") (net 35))
 (segment (start 78.5665 57.1285) (end 80.0905 58.6525) (width 0.3) (layer "B.Cu") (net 35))
 (segment (start 80.0905 58.6525) (end 86.1275 58.6525) (width 0.3) (layer "B.Cu") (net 35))
 (segment (start 77.2965 46.57185) (end 77.2965 50.5245) (width 0.3) (layer "B.Cu") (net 35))
 (segment (start 77.606175 46.262175) (end 77.2965 46.57185) (width 0.3) (layer "B.Cu") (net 35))
 (segment (start 77.8045 50.1475) (end 77.8045 53.8265) (width 0.3) (layer "F.Cu") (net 33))
 (segment (start 78.5665 49.3855) (end 77.8045 50.1475) (width 0.3) (layer "F.Cu") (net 33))
 (segment (start 77.8045 54.3345) (end 76.7885 55.3505) (width 0.3) (layer "F.Cu") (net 33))
 (segment (start 77.8045 53.8265) (end 77.8045 54.3345) (width 0.3) (layer "F.Cu") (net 33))
 (segment (start 82.4945 46.7575) (end 81.1945 46.7575) (width 0.3) (layer "F.Cu") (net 33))
 (segment (start 81.1945 46.7575) (end 78.5665 49.3855) (width 0.3) (layer "F.Cu") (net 33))
 (via (at 76.7885 55.3505) (size 1.5) (drill 0.5) (layers "F.Cu" "B.Cu") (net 33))
 (segment (start 77.0425 49.6395) (end 76.5345 50.1475) (width 0.3) (layer "F.Cu") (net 34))
 (segment (start 75.2645 54.0805) (end 75.0105 54.0805) (width 0.3) (layer "F.Cu") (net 34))
 (segment (start 76.5345 52.8105) (end 75.2645 54.0805) (width 0.3) (layer "F.Cu") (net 34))
 (segment (start 81.1945 45.4875) (end 77.0425 49.6395) (width 0.3) (layer "F.Cu") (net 34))
 (segment (start 76.5345 50.1475) (end 76.5345 52.8105) (width 0.3) (layer "F.Cu") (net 34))
 (segment (start 82.4945 45.4875) (end 81.1945 45.4875) (width 0.3) (layer "F.Cu") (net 34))
 (via (at 75.0105 54.0805) (size 1.5) (drill 0.5) (layers "F.Cu" "B.Cu") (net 34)))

